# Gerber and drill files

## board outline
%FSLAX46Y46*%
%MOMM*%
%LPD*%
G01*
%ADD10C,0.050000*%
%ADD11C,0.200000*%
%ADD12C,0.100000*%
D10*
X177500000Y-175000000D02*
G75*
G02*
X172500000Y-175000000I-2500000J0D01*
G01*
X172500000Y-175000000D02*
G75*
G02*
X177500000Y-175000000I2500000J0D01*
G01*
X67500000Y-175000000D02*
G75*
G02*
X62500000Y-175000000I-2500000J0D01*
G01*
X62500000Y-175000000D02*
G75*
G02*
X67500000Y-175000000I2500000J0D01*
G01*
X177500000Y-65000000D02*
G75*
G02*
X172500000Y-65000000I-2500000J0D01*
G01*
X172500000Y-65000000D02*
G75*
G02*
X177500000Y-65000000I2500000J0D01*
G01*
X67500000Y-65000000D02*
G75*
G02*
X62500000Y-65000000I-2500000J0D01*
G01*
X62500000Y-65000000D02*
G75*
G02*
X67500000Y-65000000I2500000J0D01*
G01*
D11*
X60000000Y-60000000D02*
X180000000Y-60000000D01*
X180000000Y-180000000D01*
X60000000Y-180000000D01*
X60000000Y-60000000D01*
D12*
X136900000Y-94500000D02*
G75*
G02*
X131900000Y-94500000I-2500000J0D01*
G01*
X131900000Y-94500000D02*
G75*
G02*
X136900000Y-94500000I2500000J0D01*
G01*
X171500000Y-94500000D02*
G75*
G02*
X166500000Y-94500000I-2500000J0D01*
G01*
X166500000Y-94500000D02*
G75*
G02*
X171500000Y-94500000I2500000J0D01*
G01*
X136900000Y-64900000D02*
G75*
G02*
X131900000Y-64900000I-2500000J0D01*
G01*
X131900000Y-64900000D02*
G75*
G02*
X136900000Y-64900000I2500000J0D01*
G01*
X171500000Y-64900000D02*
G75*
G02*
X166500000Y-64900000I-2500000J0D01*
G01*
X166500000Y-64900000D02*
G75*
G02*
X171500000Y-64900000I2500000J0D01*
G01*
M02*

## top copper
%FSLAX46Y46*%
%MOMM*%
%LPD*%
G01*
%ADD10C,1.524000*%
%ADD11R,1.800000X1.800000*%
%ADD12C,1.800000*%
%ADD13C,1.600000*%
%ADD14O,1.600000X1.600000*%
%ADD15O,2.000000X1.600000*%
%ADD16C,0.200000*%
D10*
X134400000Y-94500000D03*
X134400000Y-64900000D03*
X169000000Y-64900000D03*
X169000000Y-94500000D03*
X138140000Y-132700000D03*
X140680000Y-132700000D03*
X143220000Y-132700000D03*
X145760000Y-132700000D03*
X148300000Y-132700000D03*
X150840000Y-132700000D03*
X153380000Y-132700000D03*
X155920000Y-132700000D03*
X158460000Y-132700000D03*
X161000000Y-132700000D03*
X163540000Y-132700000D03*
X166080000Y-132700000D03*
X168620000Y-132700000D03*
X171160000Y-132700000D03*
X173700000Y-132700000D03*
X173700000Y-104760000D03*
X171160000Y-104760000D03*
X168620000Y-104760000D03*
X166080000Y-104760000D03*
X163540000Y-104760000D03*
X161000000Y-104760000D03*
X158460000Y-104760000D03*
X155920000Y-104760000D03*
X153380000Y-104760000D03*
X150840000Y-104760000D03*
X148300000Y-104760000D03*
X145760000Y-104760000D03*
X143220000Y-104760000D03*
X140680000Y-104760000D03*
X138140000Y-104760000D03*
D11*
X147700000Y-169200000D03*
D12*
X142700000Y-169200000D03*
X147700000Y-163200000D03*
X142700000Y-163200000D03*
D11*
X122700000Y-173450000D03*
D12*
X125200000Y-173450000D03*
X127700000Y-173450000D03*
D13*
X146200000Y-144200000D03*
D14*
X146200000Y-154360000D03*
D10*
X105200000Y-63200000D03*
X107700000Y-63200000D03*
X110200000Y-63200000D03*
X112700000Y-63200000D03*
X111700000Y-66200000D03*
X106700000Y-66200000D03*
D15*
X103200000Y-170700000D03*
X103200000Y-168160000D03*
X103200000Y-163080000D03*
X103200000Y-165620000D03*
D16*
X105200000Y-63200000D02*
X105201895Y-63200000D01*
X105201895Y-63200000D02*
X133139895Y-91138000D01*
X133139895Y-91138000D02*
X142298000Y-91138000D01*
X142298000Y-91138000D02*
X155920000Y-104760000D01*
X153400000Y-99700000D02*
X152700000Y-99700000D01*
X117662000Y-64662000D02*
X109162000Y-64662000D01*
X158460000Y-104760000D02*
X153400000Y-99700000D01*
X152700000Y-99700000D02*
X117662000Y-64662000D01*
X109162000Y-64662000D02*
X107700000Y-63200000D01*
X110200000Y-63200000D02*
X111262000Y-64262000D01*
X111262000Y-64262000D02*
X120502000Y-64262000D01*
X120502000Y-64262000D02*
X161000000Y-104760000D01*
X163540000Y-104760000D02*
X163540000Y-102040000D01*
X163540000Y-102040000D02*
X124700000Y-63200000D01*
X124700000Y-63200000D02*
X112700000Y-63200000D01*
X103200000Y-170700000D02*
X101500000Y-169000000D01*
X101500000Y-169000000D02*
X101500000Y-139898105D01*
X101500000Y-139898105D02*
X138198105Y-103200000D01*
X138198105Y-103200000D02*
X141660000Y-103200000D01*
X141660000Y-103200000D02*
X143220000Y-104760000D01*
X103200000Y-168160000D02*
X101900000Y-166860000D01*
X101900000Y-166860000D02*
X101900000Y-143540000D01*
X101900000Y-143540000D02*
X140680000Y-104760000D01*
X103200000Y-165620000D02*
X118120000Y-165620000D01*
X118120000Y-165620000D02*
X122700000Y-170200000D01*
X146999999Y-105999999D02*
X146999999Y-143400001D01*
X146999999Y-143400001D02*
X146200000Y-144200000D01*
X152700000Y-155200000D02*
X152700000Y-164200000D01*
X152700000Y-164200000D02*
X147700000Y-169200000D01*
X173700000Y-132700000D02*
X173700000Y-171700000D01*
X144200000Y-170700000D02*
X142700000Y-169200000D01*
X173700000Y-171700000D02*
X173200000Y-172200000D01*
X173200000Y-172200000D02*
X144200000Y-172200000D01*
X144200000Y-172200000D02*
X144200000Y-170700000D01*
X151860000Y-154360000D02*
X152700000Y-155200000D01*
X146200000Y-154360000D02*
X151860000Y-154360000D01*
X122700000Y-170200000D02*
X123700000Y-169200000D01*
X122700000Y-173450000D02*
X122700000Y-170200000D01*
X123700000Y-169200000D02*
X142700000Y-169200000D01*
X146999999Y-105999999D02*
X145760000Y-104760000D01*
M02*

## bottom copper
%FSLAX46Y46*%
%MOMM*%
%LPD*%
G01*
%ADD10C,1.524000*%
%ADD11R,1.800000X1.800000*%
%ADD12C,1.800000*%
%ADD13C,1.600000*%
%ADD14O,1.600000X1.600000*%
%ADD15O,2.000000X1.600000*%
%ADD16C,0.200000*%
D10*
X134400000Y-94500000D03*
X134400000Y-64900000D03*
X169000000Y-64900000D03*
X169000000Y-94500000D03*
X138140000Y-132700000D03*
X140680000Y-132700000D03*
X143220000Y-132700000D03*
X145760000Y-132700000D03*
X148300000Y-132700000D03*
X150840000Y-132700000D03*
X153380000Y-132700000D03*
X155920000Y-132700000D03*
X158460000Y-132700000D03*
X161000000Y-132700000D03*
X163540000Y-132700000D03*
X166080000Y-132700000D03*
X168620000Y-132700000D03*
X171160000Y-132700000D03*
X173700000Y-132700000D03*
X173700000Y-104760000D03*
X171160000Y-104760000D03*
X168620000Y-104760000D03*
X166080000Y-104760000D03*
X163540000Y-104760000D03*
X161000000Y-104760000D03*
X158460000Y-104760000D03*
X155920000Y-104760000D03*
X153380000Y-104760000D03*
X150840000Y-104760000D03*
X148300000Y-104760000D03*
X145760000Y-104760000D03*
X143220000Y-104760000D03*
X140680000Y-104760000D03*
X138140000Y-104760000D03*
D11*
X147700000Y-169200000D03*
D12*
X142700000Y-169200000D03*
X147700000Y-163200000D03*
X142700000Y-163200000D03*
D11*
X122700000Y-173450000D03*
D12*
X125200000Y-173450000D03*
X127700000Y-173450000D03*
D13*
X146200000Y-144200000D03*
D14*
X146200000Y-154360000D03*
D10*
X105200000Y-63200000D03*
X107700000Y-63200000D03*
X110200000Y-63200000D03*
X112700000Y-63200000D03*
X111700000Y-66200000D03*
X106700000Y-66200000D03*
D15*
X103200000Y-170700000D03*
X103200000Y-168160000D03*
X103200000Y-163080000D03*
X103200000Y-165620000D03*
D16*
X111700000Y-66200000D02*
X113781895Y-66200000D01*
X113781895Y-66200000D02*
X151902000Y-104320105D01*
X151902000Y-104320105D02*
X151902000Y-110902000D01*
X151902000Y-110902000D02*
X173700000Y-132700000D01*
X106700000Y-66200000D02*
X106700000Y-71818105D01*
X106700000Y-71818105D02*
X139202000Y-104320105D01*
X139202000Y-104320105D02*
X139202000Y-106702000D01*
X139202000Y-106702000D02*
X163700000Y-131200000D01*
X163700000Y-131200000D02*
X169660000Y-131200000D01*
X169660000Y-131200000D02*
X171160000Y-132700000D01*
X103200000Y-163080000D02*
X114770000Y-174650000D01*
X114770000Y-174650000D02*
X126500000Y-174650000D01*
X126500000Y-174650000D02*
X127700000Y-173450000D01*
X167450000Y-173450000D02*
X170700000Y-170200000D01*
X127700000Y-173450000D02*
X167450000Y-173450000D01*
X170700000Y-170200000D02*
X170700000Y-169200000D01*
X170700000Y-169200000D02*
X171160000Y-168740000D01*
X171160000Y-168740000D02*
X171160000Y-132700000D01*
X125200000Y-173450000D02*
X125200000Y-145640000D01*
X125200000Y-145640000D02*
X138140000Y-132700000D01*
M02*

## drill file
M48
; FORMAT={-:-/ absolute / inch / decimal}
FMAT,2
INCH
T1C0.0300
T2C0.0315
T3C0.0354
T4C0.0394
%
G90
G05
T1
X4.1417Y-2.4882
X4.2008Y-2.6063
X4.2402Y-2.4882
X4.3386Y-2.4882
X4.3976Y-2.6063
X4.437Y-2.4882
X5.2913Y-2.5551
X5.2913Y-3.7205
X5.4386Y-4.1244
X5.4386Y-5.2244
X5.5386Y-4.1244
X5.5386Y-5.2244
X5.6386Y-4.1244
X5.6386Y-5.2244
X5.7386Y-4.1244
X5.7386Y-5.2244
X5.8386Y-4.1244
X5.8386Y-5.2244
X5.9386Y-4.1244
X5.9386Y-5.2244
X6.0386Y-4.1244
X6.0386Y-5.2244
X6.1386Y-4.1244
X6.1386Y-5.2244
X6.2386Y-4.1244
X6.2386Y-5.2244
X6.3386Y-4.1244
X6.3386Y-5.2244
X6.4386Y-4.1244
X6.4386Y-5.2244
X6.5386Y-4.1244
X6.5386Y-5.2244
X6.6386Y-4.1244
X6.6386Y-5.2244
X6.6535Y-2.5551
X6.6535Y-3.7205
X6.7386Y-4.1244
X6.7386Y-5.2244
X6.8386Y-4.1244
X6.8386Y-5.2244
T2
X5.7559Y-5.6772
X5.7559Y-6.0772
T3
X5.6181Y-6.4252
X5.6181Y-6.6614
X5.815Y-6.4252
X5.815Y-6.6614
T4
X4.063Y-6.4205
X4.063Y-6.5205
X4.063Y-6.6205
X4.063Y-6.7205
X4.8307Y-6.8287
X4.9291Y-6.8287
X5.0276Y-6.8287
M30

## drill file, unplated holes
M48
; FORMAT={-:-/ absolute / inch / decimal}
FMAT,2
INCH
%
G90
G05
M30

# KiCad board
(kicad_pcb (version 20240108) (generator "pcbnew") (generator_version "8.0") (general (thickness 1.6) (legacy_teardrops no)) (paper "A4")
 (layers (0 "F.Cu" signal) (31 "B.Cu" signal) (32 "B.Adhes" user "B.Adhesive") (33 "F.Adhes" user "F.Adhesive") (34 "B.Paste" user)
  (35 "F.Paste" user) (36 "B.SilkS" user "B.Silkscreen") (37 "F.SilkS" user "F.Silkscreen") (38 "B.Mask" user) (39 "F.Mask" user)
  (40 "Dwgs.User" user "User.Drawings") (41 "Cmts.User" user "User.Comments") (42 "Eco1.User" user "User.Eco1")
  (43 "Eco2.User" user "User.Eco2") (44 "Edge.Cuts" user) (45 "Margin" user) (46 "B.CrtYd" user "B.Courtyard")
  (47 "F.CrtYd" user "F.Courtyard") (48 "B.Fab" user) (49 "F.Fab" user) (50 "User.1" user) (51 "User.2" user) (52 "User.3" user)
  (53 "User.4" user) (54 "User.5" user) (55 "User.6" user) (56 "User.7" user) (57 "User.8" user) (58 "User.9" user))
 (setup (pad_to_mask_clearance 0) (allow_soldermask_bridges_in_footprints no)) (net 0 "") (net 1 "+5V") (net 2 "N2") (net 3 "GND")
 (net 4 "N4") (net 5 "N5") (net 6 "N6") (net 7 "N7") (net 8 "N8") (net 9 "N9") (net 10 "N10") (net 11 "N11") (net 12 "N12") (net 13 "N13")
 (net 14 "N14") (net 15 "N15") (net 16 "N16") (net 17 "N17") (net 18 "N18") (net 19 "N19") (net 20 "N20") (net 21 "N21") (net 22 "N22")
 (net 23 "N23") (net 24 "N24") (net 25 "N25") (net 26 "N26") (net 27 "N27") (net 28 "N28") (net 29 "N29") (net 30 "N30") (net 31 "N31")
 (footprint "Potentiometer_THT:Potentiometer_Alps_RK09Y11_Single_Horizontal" (layer "F.Cu") (at 122.7 173.45 90)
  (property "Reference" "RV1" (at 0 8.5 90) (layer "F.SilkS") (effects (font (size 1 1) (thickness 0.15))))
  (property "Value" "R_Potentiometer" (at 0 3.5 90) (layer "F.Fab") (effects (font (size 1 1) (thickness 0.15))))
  (pad "1" thru_hole rect (at 0 0 270) (size 1.8 1.8) (drill 1) (layers "*.Cu" "*.Mask") (remove_unused_layers no) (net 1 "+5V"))
  (pad "2" thru_hole circle (at 0 2.5 270) (size 1.8 1.8) (drill 1) (layers "*.Cu" "*.Mask") (remove_unused_layers no) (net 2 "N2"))
  (pad "3" thru_hole circle (at 0 5 270) (size 1.8 1.8) (drill 1) (layers "*.Cu" "*.Mask") (remove_unused_layers no) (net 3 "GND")))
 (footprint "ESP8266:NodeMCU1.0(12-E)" (layer "F.Cu") (at 155.92 118.73 90)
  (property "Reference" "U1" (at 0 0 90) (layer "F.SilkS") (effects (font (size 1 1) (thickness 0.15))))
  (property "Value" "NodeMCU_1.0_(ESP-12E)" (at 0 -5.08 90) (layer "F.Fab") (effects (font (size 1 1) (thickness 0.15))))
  (pad "1" thru_hole circle (at -13.97 -17.78 90) (size 1.524 1.524) (drill 0.762) (layers "*.Cu" "*.Mask" "F.SilkS")
   (remove_unused_layers no) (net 2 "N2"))
  (pad "2" thru_hole circle (at -13.97 -15.24 90) (size 1.524 1.524) (drill 0.762) (layers "*.Cu" "*.Mask" "F.SilkS")
   (remove_unused_layers no) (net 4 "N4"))
  (pad "3" thru_hole circle (at -13.97 -12.7 90) (size 1.524 1.524) (drill 0.762) (layers "*.Cu" "*.Mask" "F.SilkS")
   (remove_unused_layers no) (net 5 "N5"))
  (pad "4" thru_hole circle (at -13.97 -10.16 90) (size 1.524 1.524) (drill 0.762) (layers "*.Cu" "*.Mask" "F.SilkS")
   (remove_unused_layers no) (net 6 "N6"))
  (pad "5" thru_hole circle (at -13.97 -7.62 90) (size 1.524 1.524) (drill 0.762) (layers "*.Cu" "*.Mask" "F.SilkS")
   (remove_unused_layers no) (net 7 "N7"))
  (pad "6" thru_hole circle (at -13.97 -5.08 90) (size 1.524 1.524) (drill 0.762) (layers "*.Cu" "*.Mask" "F.SilkS")
   (remove_unused_layers no) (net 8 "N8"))
  (pad "7" thru_hole circle (at -13.97 -2.54 90) (size 1.524 1.524) (drill 0.762) (layers "*.Cu" "*.Mask" "F.SilkS")
   (remove_unused_layers no) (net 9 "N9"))
  (pad "8" thru_hole circle (at -13.97 0 90) (size 1.524 1.524) (drill 0.762) (layers "*.Cu" "*.Mask" "F.SilkS") (remove_unused_layers no)
   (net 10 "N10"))
  (pad "9" thru_hole circle (at -13.97 2.54 90) (size 1.524 1.524) (drill 0.762) (layers "*.Cu" "*.Mask" "F.SilkS")
   (remove_unused_layers no) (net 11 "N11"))
  (pad "10" thru_hole circle (at -13.97 5.08 90) (size 1.524 1.524) (drill 0.762) (layers "*.Cu" "*.Mask" "F.SilkS")
   (remove_unused_layers no) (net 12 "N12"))
  (pad "11" thru_hole circle (at -13.97 7.62 90) (size 1.524 1.524) (drill 0.762) (layers "*.Cu" "*.Mask" "F.SilkS")
   (remove_unused_layers no) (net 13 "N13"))
  (pad "12" thru_hole circle (at -13.97 10.16 90) (size 1.524 1.524) (drill 0.762) (layers "*.Cu" "*.Mask" "F.SilkS")
   (remove_unused_layers no) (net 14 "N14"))
  (pad "13" thru_hole circle (at -13.97 12.7 90) (size 1.524 1.524) (drill 0.762) (layers "*.Cu" "*.Mask" "F.SilkS")
   (remove_unused_layers no) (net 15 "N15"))
  (pad "14" thru_hole circle (at -13.97 15.24 90) (size 1.524 1.524) (drill 0.762) (layers "*.Cu" "*.Mask" "F.SilkS")
   (remove_unused_layers no) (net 3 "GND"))
  (pad "15" thru_hole circle (at -13.97 17.78 90) (size 1.524 1.524) (drill 0.762) (layers "*.Cu" "*.Mask" "F.SilkS")
   (remove_unused_layers no) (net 1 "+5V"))
  (pad "16" thru_hole circle (at 13.97 17.78 90) (size 1.524 1.524) (drill 0.762) (layers "*.Cu" "*.Mask" "F.SilkS")
   (remove_unused_layers no) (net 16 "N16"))
  (pad "17" thru_hole circle (at 13.97 15.24 90) (size 1.524 1.524) (drill 0.762) (layers "*.Cu" "*.Mask" "F.SilkS")
   (remove_unused_layers no) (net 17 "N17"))
  (pad "18" thru_hole circle (at 13.97 12.7 90) (size 1.524 1.524) (drill 0.762) (layers "*.Cu" "*.Mask" "F.SilkS")
   (remove_unused_layers no) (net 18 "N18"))
  (pad "19" thru_hole circle (at 13.97 10.16 90) (size 1.524 1.524) (drill 0.762) (layers "*.Cu" "*.Mask" "F.SilkS")
   (remove_unused_layers no) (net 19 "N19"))
  (pad "20" thru_hole circle (at 13.97 7.62 90) (size 1.524 1.524) (drill 0.762) (layers "*.Cu" "*.Mask" "F.SilkS")
   (remove_unused_layers no) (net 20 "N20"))
  (pad "21" thru_hole circle (at 13.97 5.08 90) (size 1.524 1.524) (drill 0.762) (layers "*.Cu" "*.Mask" "F.SilkS")
   (remove_unused_layers no) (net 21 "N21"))
  (pad "22" thru_hole circle (at 13.97 2.54 90) (size 1.524 1.524) (drill 0.762) (layers "*.Cu" "*.Mask" "F.SilkS")
   (remove_unused_layers no) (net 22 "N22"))
  (pad "23" thru_hole circle (at 13.97 0 90) (size 1.524 1.524) (drill 0.762) (layers "*.Cu" "*.Mask" "F.SilkS") (remove_unused_layers no)
   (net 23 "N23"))
  (pad "24" thru_hole circle (at 13.97 -2.54 90) (size 1.524 1.524) (drill 0.762) (layers "*.Cu" "*.Mask" "F.SilkS")
   (remove_unused_layers no) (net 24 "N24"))
  (pad "25" thru_hole circle (at 13.97 -5.08 90) (size 1.524 1.524) (drill 0.762) (layers "*.Cu" "*.Mask" "F.SilkS")
   (remove_unused_layers no) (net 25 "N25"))
  (pad "26" thru_hole circle (at 13.97 -7.62 90) (size 1.524 1.524) (drill 0.762) (layers "*.Cu" "*.Mask" "F.SilkS")
   (remove_unused_layers no) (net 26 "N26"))
  (pad "27" thru_hole circle (at 13.97 -10.16 90) (size 1.524 1.524) (drill 0.762) (layers "*.Cu" "*.Mask" "F.SilkS")
   (remove_unused_layers no) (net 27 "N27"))
  (pad "28" thru_hole circle (at 13.97 -12.7 90) (size 1.524 1.524) (drill 0.762) (layers "*.Cu" "*.Mask" "F.SilkS")
   (remove_unused_layers no) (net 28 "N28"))
  (pad "29" thru_hole circle (at 13.97 -15.24 90) (size 1.524 1.524) (drill 0.762) (layers "*.Cu" "*.Mask" "F.SilkS")
   (remove_unused_layers no) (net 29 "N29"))
  (pad "30" thru_hole circle (at 13.97 -17.78 90) (size 1.524 1.524) (drill 0.762) (layers "*.Cu" "*.Mask" "F.SilkS")
   (remove_unused_layers no) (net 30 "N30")))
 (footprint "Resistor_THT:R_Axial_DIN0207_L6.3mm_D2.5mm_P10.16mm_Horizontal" (layer "F.Cu") (at 146.2 144.2 -90)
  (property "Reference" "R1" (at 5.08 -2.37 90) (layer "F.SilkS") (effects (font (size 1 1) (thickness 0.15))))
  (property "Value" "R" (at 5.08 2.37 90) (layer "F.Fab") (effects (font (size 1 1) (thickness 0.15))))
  (pad "1" thru_hole circle (at 0 0 270) (size 1.6 1.6) (drill 0.8) (layers "*.Cu" "*.Mask") (remove_unused_layers no) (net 27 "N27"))
  (pad "2" thru_hole oval (at 10.16 0 270) (size 1.6 1.6) (drill 0.8) (layers "*.Cu" "*.Mask") (remove_unused_layers no) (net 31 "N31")))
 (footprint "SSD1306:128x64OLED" (layer "F.Cu") (at 92.6 166.7 -90)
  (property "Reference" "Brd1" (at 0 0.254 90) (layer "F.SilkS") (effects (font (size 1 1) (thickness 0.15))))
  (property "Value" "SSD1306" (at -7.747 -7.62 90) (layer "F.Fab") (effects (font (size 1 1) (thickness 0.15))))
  (pad "1" thru_hole oval (at -3.62 -10.6) (size 2 1.6) (drill 1) (layers "*.Cu" "*.Mask") (remove_unused_layers no) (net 3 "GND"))
  (pad "2" thru_hole oval (at -1.08 -10.6) (size 2 1.6) (drill 1) (layers "*.Cu" "*.Mask") (remove_unused_layers no) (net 1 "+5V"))
  (pad "3" thru_hole oval (at 1.46 -10.6) (size 2 1.6) (drill 1) (layers "*.Cu" "*.Mask") (remove_unused_layers no) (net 29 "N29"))
  (pad "4" thru_hole oval (at 4 -10.6) (size 2 1.6) (drill 1) (layers "*.Cu" "*.Mask") (remove_unused_layers no) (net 28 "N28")))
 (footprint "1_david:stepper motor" (layer "F.Cu") (at 111.7 63.2)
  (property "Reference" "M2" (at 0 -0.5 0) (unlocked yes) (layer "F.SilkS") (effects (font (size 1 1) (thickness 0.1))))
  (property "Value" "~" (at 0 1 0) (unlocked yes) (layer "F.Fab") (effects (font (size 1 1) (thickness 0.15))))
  (pad "1" thru_hole circle (at -6.5 0) (size 1.524 1.524) (drill 0.762) (layers "*.Cu" "*.Mask") (remove_unused_layers no) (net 23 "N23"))
  (pad "2" thru_hole circle (at -4 0) (size 1.524 1.524) (drill 0.762) (layers "*.Cu" "*.Mask") (remove_unused_layers no) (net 22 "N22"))
  (pad "3" thru_hole circle (at -1.5 0) (size 1.524 1.524) (drill 0.762) (layers "*.Cu" "*.Mask") (remove_unused_layers no) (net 21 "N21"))
  (pad "4" thru_hole circle (at 1 0) (size 1.524 1.524) (drill 0.762) (layers "*.Cu" "*.Mask") (remove_unused_layers no) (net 20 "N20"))
  (pad "5" thru_hole circle (at 0 3) (size 1.524 1.524) (drill 0.762) (layers "*.Cu" "*.Mask") (remove_unused_layers no) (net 1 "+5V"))
  (pad "6" thru_hole circle (at -5 3) (size 1.524 1.524) (drill 0.762) (layers "*.Cu" "*.Mask") (remove_unused_layers no) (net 3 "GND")))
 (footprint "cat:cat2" (layer "F.Cu") (at 87.5 103)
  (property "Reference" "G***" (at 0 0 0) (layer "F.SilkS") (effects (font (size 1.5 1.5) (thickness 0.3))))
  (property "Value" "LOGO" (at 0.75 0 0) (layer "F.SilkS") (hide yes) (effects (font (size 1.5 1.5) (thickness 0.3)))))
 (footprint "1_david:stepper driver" (layer "F.Cu") (at 142.4 87 90)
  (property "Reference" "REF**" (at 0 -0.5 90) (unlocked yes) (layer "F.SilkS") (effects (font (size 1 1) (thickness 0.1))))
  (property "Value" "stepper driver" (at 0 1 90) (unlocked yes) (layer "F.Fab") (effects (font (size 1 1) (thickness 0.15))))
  (fp_circle (center 22.1 -8) (end 24.6 -8) (stroke (width 0.1) (type default)) (fill none) (layer "Edge.Cuts"))
  (fp_circle (center -7.5 -8) (end -5 -8) (stroke (width 0.1) (type default)) (fill none) (layer "Edge.Cuts"))
  (fp_circle (center 22.1 26.6) (end 24.6 26.6) (stroke (width 0.1) (type default)) (fill none) (layer "Edge.Cuts"))
  (fp_circle (center -7.5 26.6) (end -5 26.6) (stroke (width 0.1) (type default)) (fill none) (layer "Edge.Cuts"))
  (pad "1" thru_hole circle (at -7.5 -8 90) (size 1.524 1.524) (drill 0.762) (layers "*.Cu" "*.Mask") (remove_unused_layers no))
  (pad "2" thru_hole circle (at 22.1 -8 90) (size 1.524 1.524) (drill 0.762) (layers "*.Cu" "*.Mask") (remove_unused_layers no))
  (pad "3" thru_hole circle (at 22.1 26.6 90) (size 1.524 1.524) (drill 0.762) (layers "*.Cu" "*.Mask") (remove_unused_layers no))
  (pad "4" thru_hole circle (at -7.5 26.6 90) (size 1.524 1.524) (drill 0.762) (layers "*.Cu" "*.Mask") (remove_unused_layers no)))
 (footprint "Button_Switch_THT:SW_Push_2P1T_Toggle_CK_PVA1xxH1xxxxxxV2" (layer "F.Cu") (at 147.7 169.2 180)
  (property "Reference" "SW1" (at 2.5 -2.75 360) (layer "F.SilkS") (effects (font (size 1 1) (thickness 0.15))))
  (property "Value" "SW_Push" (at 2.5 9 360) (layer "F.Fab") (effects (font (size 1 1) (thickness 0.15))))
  (pad "1" thru_hole rect (at 0 0 180) (size 1.8 1.8) (drill 0.9) (layers "*.Cu" "*.Mask") (remove_unused_layers no) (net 31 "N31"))
  (pad "2" thru_hole circle (at 5 0 180) (size 1.8 1.8) (drill 0.9) (layers "*.Cu" "*.Mask") (remove_unused_layers no) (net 1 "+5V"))
  (pad "3" thru_hole circle (at 0 6 180) (size 1.8 1.8) (drill 0.9) (layers "*.Cu" "*.Mask") (remove_unused_layers no))
  (pad "4" thru_hole circle (at 5 6 180) (size 1.8 1.8) (drill 0.9) (layers "*.Cu" "*.Mask") (remove_unused_layers no)))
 (gr_circle (center 65 65) (end 67.5 65) (stroke (width 0.05) (type default)) (fill none) (layer "Edge.Cuts"))
 (gr_circle (center 175 175) (end 177.5 175) (stroke (width 0.05) (type default)) (fill none) (layer "Edge.Cuts"))
 (gr_rect (start 60 60) (end 180 180) (stroke (width 0.2) (type default)) (fill none) (layer "Edge.Cuts"))
 (gr_circle (center 175 65) (end 177.5 65) (stroke (width 0.05) (type default)) (fill none) (layer "Edge.Cuts"))
 (gr_circle (center 65 175) (end 67.5 175) (stroke (width 0.05) (type default)) (fill none) (layer "Edge.Cuts"))
 (segment (start 122.7 173.45) (end 122.7 170.2) (width 0.2) (layer "F.Cu") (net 1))
 (segment (start 173.7 171.7) (end 173.2 172.2) (width 0.2) (layer "F.Cu") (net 1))
 (segment (start 122.7 170.2) (end 123.7 169.2) (width 0.2) (layer "F.Cu") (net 1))
 (segment (start 144.2 170.7) (end 142.7 169.2) (width 0.2) (layer "F.Cu") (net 1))
 (segment (start 123.7 169.2) (end 142.7 169.2) (width 0.2) (layer "F.Cu") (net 1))
 (segment (start 173.2 172.2) (end 144.2 172.2) (width 0.2) (layer "F.Cu") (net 1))
 (segment (start 144.2 172.2) (end 144.2 170.7) (width 0.2) (layer "F.Cu") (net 1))
 (segment (start 103.2 165.62) (end 118.12 165.62) (width 0.2) (layer "F.Cu") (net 1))
 (segment (start 173.7 132.7) (end 173.7 171.7) (width 0.2) (layer "F.Cu") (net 1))
 (segment (start 118.12 165.62) (end 122.7 170.2) (width 0.2) (layer "F.Cu") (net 1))
 (segment (start 111.7 66.2) (end 113.781895 66.2) (width 0.2) (layer "B.Cu") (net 1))
 (segment (start 113.781895 66.2) (end 151.902 104.320105) (width 0.2) (layer "B.Cu") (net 1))
 (segment (start 151.902 104.320105) (end 151.902 110.902) (width 0.2) (layer "B.Cu") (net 1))
 (segment (start 151.902 110.902) (end 173.7 132.7) (width 0.2) (layer "B.Cu") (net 1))
 (segment (start 139.202 106.702) (end 163.7 131.2) (width 0.2) (layer "B.Cu") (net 3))
 (segment (start 106.7 66.2) (end 106.7 71.818105) (width 0.2) (layer "B.Cu") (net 3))
 (segment (start 106.7 71.818105) (end 139.202 104.320105) (width 0.2) (layer "B.Cu") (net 3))
 (segment (start 170.7 169.2) (end 171.16 168.74) (width 0.2) (layer "B.Cu") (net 3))
 (segment (start 169.66 131.2) (end 171.16 132.7) (width 0.2) (layer "B.Cu") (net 3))
 (segment (start 126.5 174.65) (end 127.7 173.45) (width 0.2) (layer "B.Cu") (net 3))
 (segment (start 114.77 174.65) (end 126.5 174.65) (width 0.2) (layer "B.Cu") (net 3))
 (segment (start 127.7 173.45) (end 167.45 173.45) (width 0.2) (layer "B.Cu") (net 3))
 (segment (start 139.202 104.320105) (end 139.202 106.702) (width 0.2) (layer "B.Cu") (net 3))
 (segment (start 167.45 173.45) (end 170.7 170.2) (width 0.2) (layer "B.Cu") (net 3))
 (segment (start 163.7 131.2) (end 169.66 131.2) (width 0.2) (layer "B.Cu") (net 3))
 (segment (start 103.2 163.08) (end 114.77 174.65) (width 0.2) (layer "B.Cu") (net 3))
 (segment (start 171.16 168.74) (end 171.16 132.7) (width 0.2) (layer "B.Cu") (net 3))
 (segment (start 170.7 170.2) (end 170.7 169.2) (width 0.2) (layer "B.Cu") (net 3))
 (segment (start 101.5 169) (end 101.5 139.898105) (width 0.2) (layer "F.Cu") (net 28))
 (segment (start 138.198105 103.2) (end 141.66 103.2) (width 0.2) (layer "F.Cu") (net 28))
 (segment (start 141.66 103.2) (end 143.22 104.76) (width 0.2) (layer "F.Cu") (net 28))
 (segment (start 103.2 170.7) (end 101.5 169) (width 0.2) (layer "F.Cu") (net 28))
 (segment (start 101.5 139.898105) (end 138.198105 103.2) (width 0.2) (layer "F.Cu") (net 28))
 (segment (start 101.9 166.86) (end 101.9 143.54) (width 0.2) (layer "F.Cu") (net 29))
 (segment (start 101.9 143.54) (end 140.68 104.76) (width 0.2) (layer "F.Cu") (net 29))
 (segment (start 103.2 168.16) (end 101.9 166.86) (width 0.2) (layer "F.Cu") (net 29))
 (segment (start 146.999999 105.999999) (end 145.76 104.76) (width 0.2) (layer "F.Cu") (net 27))
 (segment (start 146.999999 105.999999) (end 146.999999 143.400001) (width 0.2) (layer "F.Cu") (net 27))
 (segment (start 146.999999 143.400001) (end 146.2 144.2) (width 0.2) (layer "F.Cu") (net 27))
 (segment (start 151.86 154.36) (end 152.7 155.2) (width 0.2) (layer "F.Cu") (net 31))
 (segment (start 146.2 154.36) (end 151.86 154.36) (width 0.2) (layer "F.Cu") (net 31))
 (segment (start 152.7 155.2) (end 152.7 164.2) (width 0.2) (layer "F.Cu") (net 31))
 (segment (start 152.7 164.2) (end 147.7 169.2) (width 0.2) (layer "F.Cu") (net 31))
 (segment (start 125.2 145.64) (end 138.14 132.7) (width 0.2) (layer "B.Cu") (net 2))
 (segment (start 125.2 173.45) (end 125.2 145.64) (width 0.2) (layer "B.Cu") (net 2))
 (segment (start 105.2 63.2) (end 105.201895 63.2) (width 0.2) (layer "F.Cu") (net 23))
 (segment (start 105.201895 63.2) (end 133.139895 91.138) (width 0.2) (layer "F.Cu") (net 23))
 (segment (start 142.298 91.138) (end 155.92 104.76) (width 0.2) (layer "F.Cu") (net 23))
 (segment (start 133.139895 91.138) (end 142.298 91.138) (width 0.2) (layer "F.Cu") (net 23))
 (segment (start 163.54 104.76) (end 163.54 102.04) (width 0.2) (layer "F.Cu") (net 20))
 (segment (start 163.54 102.04) (end 124.7 63.2) (width 0.2) (layer "F.Cu") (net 20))
 (segment (start 124.7 63.2) (end 112.7 63.2) (width 0.2) (layer "F.Cu") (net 20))
 (segment (start 152.7 99.7) (end 117.662 64.662) (width 0.2) (layer "F.Cu") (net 22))
 (segment (start 109.162 64.662) (end 107.7 63.2) (width 0.2) (layer "F.Cu") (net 22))
 (segment (start 117.662 64.662) (end 109.162 64.662) (width 0.2) (layer "F.Cu") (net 22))
 (segment (start 158.46 104.76) (end 153.4 99.7) (width 0.2) (layer "F.Cu") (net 22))
 (segment (start 153.4 99.7) (end 152.7 99.7) (width 0.2) (layer "F.Cu") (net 22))
 (segment (start 110.2 63.2) (end 111.262 64.262) (width 0.2) (layer "F.Cu") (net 21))
 (segment (start 111.262 64.262) (end 120.502 64.262) (width 0.2) (layer "F.Cu") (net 21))
 (segment (start 120.502 64.262) (end 161 104.76) (width 0.2) (layer "F.Cu") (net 21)))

